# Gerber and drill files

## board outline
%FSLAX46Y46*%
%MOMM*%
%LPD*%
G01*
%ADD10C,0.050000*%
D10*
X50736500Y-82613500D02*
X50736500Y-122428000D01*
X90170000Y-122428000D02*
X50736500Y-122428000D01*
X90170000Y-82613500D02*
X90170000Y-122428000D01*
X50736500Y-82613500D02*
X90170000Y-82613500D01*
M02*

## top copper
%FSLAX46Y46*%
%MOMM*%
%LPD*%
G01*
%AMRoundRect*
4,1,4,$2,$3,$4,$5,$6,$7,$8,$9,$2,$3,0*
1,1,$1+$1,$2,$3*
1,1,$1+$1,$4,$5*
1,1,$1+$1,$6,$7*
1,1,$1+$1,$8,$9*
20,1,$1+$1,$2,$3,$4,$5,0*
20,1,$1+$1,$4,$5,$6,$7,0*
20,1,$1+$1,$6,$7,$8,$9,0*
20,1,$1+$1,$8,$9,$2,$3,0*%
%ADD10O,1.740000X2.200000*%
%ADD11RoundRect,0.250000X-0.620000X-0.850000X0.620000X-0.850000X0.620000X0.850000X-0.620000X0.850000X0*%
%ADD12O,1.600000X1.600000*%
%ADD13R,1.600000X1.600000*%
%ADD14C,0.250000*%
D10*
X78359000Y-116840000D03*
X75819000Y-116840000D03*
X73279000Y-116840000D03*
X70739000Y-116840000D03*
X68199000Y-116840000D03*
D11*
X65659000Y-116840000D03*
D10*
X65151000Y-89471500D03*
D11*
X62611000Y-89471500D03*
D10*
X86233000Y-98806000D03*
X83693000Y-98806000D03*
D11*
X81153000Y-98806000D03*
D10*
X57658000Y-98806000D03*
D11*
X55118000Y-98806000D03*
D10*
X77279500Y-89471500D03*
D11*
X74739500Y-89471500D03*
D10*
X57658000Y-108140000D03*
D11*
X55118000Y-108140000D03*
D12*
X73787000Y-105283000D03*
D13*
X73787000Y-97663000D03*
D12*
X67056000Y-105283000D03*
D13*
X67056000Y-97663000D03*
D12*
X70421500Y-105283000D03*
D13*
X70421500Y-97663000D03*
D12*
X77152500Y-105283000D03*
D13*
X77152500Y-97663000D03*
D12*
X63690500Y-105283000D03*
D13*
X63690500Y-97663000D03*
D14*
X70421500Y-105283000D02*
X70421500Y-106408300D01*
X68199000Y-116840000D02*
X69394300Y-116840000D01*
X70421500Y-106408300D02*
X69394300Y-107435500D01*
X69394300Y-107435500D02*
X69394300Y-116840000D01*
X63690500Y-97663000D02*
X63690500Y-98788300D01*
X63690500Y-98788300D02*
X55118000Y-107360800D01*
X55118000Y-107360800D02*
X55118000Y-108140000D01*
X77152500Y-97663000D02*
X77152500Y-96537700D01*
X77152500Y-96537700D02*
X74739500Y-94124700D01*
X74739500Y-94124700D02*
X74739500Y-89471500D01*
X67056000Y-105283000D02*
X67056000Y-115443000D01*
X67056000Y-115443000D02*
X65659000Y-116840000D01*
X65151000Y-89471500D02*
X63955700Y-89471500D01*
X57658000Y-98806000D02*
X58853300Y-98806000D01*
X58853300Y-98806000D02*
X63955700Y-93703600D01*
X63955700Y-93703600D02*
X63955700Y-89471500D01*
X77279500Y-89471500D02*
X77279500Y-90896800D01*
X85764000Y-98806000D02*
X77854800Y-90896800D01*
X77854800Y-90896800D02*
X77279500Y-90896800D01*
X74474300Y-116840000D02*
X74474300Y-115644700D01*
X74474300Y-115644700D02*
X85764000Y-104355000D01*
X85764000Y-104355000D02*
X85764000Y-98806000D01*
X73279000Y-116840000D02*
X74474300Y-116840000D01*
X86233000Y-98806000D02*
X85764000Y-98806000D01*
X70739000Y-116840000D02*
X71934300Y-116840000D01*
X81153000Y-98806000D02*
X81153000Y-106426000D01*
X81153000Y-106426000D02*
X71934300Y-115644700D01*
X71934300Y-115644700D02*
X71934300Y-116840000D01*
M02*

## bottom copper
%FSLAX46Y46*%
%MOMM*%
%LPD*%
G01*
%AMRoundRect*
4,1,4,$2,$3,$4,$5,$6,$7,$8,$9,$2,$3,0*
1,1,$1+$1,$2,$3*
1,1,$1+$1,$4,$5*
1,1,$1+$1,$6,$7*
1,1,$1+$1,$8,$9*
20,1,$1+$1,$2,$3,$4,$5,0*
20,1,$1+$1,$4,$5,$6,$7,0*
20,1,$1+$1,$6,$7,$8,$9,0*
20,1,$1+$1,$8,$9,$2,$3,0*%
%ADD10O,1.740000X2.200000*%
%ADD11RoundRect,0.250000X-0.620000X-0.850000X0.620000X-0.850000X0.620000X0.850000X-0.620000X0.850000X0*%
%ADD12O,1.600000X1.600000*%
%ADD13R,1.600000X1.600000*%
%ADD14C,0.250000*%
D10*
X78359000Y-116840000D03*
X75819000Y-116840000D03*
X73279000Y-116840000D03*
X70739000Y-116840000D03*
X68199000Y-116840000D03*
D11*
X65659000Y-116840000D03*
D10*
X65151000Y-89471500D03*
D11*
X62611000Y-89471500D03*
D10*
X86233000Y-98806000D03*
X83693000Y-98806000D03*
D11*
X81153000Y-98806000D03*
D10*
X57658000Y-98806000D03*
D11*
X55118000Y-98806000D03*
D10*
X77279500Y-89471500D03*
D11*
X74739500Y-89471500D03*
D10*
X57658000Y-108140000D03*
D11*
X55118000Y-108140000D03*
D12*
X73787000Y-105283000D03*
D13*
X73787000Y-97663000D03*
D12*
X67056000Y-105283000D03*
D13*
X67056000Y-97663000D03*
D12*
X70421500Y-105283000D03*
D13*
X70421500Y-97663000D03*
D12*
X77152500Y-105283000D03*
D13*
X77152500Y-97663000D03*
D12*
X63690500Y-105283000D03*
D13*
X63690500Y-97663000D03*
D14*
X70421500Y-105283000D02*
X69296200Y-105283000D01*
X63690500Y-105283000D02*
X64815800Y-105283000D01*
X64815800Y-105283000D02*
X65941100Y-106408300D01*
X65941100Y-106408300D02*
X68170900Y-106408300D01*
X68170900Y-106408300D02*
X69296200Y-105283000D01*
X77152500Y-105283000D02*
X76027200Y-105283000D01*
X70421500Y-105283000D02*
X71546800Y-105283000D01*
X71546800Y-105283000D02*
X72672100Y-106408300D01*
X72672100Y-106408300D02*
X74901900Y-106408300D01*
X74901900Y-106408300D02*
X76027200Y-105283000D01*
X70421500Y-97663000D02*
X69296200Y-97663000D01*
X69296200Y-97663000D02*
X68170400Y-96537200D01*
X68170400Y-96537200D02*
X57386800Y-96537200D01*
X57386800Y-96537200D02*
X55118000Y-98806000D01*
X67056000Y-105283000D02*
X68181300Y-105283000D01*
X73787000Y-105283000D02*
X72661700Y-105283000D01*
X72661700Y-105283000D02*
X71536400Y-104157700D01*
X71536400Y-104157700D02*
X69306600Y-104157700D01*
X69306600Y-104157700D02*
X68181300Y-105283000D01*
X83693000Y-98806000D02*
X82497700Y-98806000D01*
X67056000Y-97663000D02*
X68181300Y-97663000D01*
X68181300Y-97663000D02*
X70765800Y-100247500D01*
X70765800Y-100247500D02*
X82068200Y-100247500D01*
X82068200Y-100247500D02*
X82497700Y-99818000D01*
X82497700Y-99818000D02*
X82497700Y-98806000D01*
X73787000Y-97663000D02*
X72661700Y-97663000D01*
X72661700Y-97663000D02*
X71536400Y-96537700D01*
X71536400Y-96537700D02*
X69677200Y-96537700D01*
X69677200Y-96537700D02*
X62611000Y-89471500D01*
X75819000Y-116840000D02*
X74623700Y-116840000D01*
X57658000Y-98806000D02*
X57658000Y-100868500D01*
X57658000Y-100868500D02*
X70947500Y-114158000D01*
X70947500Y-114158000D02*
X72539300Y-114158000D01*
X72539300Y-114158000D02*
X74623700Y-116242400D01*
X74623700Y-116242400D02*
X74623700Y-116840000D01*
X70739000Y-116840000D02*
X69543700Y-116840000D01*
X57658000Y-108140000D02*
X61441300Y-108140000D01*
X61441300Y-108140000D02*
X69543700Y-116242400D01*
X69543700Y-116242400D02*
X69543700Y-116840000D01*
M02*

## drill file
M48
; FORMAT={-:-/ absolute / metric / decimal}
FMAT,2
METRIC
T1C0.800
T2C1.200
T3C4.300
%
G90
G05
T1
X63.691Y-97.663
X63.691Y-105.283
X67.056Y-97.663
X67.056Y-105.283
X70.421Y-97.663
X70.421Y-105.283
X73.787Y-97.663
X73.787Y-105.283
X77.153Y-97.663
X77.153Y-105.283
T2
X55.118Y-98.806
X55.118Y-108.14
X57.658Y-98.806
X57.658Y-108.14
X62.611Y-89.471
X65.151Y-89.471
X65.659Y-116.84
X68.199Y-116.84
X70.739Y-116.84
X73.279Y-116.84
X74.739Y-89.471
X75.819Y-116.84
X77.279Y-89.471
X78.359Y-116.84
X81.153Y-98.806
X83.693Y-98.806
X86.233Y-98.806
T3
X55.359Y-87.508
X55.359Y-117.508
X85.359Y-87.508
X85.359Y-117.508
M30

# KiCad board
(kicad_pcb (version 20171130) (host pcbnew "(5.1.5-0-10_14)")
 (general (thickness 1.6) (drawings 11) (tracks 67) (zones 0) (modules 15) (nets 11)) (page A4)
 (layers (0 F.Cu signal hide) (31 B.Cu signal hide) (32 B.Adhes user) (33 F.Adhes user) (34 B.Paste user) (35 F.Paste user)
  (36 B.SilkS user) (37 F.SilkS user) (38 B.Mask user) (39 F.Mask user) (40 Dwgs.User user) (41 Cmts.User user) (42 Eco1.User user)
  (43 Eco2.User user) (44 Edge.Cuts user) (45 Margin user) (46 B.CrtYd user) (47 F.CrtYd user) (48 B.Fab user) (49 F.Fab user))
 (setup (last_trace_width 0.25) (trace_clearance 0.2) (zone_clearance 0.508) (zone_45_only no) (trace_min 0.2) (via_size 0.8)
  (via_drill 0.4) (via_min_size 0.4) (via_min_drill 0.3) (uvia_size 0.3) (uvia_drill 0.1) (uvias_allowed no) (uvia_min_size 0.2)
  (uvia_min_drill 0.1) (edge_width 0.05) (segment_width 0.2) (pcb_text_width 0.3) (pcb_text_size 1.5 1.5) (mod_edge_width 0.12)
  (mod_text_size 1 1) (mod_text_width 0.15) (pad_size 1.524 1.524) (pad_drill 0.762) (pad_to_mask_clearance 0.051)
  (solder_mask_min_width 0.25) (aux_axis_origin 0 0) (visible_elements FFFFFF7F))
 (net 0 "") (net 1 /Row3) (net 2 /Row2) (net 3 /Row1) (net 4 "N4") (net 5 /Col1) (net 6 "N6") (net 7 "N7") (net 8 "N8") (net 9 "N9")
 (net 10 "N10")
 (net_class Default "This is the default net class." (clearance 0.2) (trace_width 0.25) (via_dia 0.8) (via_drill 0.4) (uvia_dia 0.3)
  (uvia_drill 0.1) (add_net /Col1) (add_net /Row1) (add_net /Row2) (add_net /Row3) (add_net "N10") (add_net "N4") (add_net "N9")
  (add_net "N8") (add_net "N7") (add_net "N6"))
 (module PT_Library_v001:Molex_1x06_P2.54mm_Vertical (layer F.Cu) (at 65.659 116.84)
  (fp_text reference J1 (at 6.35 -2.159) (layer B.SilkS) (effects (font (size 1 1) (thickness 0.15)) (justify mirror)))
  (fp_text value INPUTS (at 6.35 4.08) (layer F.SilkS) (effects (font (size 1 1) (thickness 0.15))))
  (pad 6 thru_hole oval (at 12.7 0) (size 1.74 2.2) (drill 1.2) (layers *.Cu *.Mask))
  (pad 5 thru_hole oval (at 10.16 0) (size 1.74 2.2) (drill 1.2) (layers *.Cu *.Mask) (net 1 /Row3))
  (pad 4 thru_hole oval (at 7.62 0) (size 1.74 2.2) (drill 1.2) (layers *.Cu *.Mask) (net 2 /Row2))
  (pad 3 thru_hole oval (at 5.08 0) (size 1.74 2.2) (drill 1.2) (layers *.Cu *.Mask) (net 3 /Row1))
  (pad 2 thru_hole oval (at 2.54 0) (size 1.74 2.2) (drill 1.2) (layers *.Cu *.Mask) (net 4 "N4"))
  (pad 1 thru_hole roundrect (at 0 0) (size 1.74 2.2) (drill 1.2) (layers *.Cu *.Mask) (roundrect_rratio 0.143678) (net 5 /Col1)))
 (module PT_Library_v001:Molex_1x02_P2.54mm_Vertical (layer F.Cu) (at 62.611 89.4715)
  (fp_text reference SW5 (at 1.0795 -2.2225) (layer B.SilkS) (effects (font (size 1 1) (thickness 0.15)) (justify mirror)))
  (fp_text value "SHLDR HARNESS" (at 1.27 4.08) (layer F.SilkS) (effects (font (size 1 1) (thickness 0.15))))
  (pad 2 thru_hole oval (at 2.54 0) (size 1.74 2.2) (drill 1.2) (layers *.Cu *.Mask) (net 1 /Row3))
  (pad 1 thru_hole roundrect (at 0 0) (size 1.74 2.2) (drill 1.2) (layers *.Cu *.Mask) (roundrect_rratio 0.143678) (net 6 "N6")))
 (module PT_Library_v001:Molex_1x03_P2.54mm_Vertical (layer F.Cu) (at 81.153 98.806)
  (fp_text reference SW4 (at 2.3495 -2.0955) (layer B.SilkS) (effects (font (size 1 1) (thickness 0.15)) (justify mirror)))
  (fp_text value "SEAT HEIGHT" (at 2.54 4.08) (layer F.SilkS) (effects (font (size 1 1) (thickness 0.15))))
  (pad 3 thru_hole oval (at 5.08 0) (size 1.74 2.2) (drill 1.2) (layers *.Cu *.Mask) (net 2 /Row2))
  (pad 2 thru_hole oval (at 2.54 0) (size 1.74 2.2) (drill 1.2) (layers *.Cu *.Mask) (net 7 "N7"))
  (pad 1 thru_hole roundrect (at 0 0) (size 1.74 2.2) (drill 1.2) (layers *.Cu *.Mask) (roundrect_rratio 0.143678) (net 3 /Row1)))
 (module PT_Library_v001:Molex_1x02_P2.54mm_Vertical (layer F.Cu) (at 55.118 98.806)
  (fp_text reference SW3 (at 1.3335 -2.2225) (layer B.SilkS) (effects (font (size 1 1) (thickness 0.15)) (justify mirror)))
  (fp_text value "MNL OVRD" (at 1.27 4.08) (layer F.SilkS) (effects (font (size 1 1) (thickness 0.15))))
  (pad 2 thru_hole oval (at 2.54 0) (size 1.74 2.2) (drill 1.2) (layers *.Cu *.Mask) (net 1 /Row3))
  (pad 1 thru_hole roundrect (at 0 0) (size 1.74 2.2) (drill 1.2) (layers *.Cu *.Mask) (roundrect_rratio 0.143678) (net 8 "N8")))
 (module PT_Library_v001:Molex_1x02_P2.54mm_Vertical (layer F.Cu) (at 74.7395 89.4715)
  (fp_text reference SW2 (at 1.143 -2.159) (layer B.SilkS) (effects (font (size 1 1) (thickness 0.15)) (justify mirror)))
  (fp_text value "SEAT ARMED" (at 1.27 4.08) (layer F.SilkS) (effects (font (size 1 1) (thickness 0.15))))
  (pad 2 thru_hole oval (at 2.54 0) (size 1.74 2.2) (drill 1.2) (layers *.Cu *.Mask) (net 2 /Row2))
  (pad 1 thru_hole roundrect (at 0 0) (size 1.74 2.2) (drill 1.2) (layers *.Cu *.Mask) (roundrect_rratio 0.143678) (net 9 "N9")))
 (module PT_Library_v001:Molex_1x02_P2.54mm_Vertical (layer F.Cu) (at 55.118 108.14)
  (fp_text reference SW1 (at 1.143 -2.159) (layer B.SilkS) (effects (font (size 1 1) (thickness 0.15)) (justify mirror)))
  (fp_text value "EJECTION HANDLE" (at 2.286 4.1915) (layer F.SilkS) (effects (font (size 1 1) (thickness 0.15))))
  (pad 2 thru_hole oval (at 2.54 0) (size 1.74 2.2) (drill 1.2) (layers *.Cu *.Mask) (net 3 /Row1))
  (pad 1 thru_hole roundrect (at 0 0) (size 1.74 2.2) (drill 1.2) (layers *.Cu *.Mask) (roundrect_rratio 0.143678) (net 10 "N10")))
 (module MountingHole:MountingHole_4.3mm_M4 (layer F.Cu) (at 55.3595 117.508)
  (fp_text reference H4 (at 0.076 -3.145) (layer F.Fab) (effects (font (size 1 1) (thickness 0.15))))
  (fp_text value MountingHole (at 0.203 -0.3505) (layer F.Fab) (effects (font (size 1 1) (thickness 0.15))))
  (pad 1 np_thru_hole circle (at 0 0) (size 4.3 4.3) (drill 4.3) (layers *.Cu *.Mask)))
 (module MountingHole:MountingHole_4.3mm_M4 (layer F.Cu) (at 85.3595 117.508)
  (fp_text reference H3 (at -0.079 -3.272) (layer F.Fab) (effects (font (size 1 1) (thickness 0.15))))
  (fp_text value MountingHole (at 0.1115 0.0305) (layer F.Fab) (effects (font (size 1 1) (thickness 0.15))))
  (pad 1 np_thru_hole circle (at 0 0) (size 4.3 4.3) (drill 4.3) (layers *.Cu *.Mask)))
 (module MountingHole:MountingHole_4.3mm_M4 (layer F.Cu) (at 55.3595 87.5085)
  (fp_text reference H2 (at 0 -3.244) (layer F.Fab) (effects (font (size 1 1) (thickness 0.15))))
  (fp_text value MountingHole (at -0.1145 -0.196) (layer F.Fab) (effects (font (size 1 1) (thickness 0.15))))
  (pad 1 np_thru_hole circle (at 0 0) (size 4.3 4.3) (drill 4.3) (layers *.Cu *.Mask)))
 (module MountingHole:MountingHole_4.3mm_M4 (layer F.Cu) (at 85.3595 87.5085)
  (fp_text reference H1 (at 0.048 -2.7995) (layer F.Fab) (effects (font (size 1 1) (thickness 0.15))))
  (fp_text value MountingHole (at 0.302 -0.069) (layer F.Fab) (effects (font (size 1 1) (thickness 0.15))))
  (pad 1 np_thru_hole circle (at 0 0) (size 4.3 4.3) (drill 4.3) (layers *.Cu *.Mask)))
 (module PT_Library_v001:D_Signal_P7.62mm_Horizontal (layer F.Cu) (at 73.787 97.663 270)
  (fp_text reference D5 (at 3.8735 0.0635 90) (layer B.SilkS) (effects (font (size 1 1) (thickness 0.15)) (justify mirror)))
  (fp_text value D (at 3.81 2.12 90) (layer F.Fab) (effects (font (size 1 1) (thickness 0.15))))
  (pad 2 thru_hole oval (at 7.62 0 270) (size 1.6 1.6) (drill 0.8) (layers *.Cu *.Mask) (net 5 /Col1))
  (pad 1 thru_hole rect (at 0 0 270) (size 1.6 1.6) (drill 0.8) (layers *.Cu *.Mask) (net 6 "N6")))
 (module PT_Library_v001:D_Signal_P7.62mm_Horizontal (layer F.Cu) (at 67.056 97.663 270)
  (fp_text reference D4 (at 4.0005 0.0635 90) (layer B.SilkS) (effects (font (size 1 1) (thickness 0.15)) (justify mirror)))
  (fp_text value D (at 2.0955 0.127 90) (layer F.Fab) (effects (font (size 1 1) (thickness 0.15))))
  (pad 2 thru_hole oval (at 7.62 0 270) (size 1.6 1.6) (drill 0.8) (layers *.Cu *.Mask) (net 5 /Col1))
  (pad 1 thru_hole rect (at 0 0 270) (size 1.6 1.6) (drill 0.8) (layers *.Cu *.Mask) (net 7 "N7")))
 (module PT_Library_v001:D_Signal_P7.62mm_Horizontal (layer F.Cu) (at 70.4215 97.663 270)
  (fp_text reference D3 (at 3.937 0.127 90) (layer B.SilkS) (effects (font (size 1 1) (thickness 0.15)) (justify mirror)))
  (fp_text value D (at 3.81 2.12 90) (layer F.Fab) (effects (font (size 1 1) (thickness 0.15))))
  (pad 2 thru_hole oval (at 7.62 0 270) (size 1.6 1.6) (drill 0.8) (layers *.Cu *.Mask) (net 4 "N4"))
  (pad 1 thru_hole rect (at 0 0 270) (size 1.6 1.6) (drill 0.8) (layers *.Cu *.Mask) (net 8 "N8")))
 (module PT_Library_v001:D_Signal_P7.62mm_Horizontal (layer F.Cu) (at 77.1525 97.663 270)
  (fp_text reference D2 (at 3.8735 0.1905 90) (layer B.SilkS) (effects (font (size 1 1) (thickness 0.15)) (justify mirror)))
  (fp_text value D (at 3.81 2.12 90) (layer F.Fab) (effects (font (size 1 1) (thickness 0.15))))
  (pad 2 thru_hole oval (at 7.62 0 270) (size 1.6 1.6) (drill 0.8) (layers *.Cu *.Mask) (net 4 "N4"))
  (pad 1 thru_hole rect (at 0 0 270) (size 1.6 1.6) (drill 0.8) (layers *.Cu *.Mask) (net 9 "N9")))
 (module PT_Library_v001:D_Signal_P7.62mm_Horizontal (layer F.Cu) (at 63.6905 97.663 270)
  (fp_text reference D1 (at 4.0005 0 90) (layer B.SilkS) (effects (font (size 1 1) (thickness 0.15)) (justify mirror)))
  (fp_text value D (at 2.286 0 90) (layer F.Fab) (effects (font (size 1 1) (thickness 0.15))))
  (pad 2 thru_hole oval (at 7.62 0 270) (size 1.6 1.6) (drill 0.8) (layers *.Cu *.Mask) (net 4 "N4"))
  (pad 1 thru_hole rect (at 0 0 270) (size 1.6 1.6) (drill 0.8) (layers *.Cu *.Mask) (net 10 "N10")))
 (gr_line (start 50.7365 82.6135) (end 50.7365 122.428) (layer Edge.Cuts) (width 0.05))
 (gr_line (start 90.17 122.428) (end 50.7365 122.428) (layer Edge.Cuts) (width 0.05))
 (gr_line (start 90.17 82.6135) (end 90.17 122.428) (layer Edge.Cuts) (width 0.05))
 (gr_line (start 50.7365 82.6135) (end 90.17 82.6135) (layer Edge.Cuts) (width 0.05))
 (segment (start 70.4215 105.283) (end 69.2962 105.283) (width 0.25) (layer B.Cu) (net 4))
 (segment (start 63.6905 105.283) (end 64.8158 105.283) (width 0.25) (layer B.Cu) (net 4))
 (segment (start 64.8158 105.283) (end 65.9411 106.4083) (width 0.25) (layer B.Cu) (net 4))
 (segment (start 65.9411 106.4083) (end 68.1709 106.4083) (width 0.25) (layer B.Cu) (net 4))
 (segment (start 68.1709 106.4083) (end 69.2962 105.283) (width 0.25) (layer B.Cu) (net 4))
 (segment (start 77.1525 105.283) (end 76.0272 105.283) (width 0.25) (layer B.Cu) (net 4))
 (segment (start 70.4215 105.283) (end 71.5468 105.283) (width 0.25) (layer B.Cu) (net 4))
 (segment (start 71.5468 105.283) (end 72.6721 106.4083) (width 0.25) (layer B.Cu) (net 4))
 (segment (start 72.6721 106.4083) (end 74.9019 106.4083) (width 0.25) (layer B.Cu) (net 4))
 (segment (start 74.9019 106.4083) (end 76.0272 105.283) (width 0.25) (layer B.Cu) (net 4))
 (segment (start 70.4215 105.283) (end 70.4215 106.4083) (width 0.25) (layer F.Cu) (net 4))
 (segment (start 68.199 116.84) (end 69.3943 116.84) (width 0.25) (layer F.Cu) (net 4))
 (segment (start 70.4215 106.4083) (end 69.3943 107.4355) (width 0.25) (layer F.Cu) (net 4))
 (segment (start 69.3943 107.4355) (end 69.3943 116.84) (width 0.25) (layer F.Cu) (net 4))
 (segment (start 63.6905 97.663) (end 63.6905 98.7883) (width 0.25) (layer F.Cu) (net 10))
 (segment (start 63.6905 98.7883) (end 55.118 107.3608) (width 0.25) (layer F.Cu) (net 10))
 (segment (start 55.118 107.3608) (end 55.118 108.14) (width 0.25) (layer F.Cu) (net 10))
 (segment (start 77.1525 97.663) (end 77.1525 96.5377) (width 0.25) (layer F.Cu) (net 9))
 (segment (start 77.1525 96.5377) (end 74.7395 94.1247) (width 0.25) (layer F.Cu) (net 9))
 (segment (start 74.7395 94.1247) (end 74.7395 89.4715) (width 0.25) (layer F.Cu) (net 9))
 (segment (start 70.4215 97.663) (end 69.2962 97.663) (width 0.25) (layer B.Cu) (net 8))
 (segment (start 69.2962 97.663) (end 68.1704 96.5372) (width 0.25) (layer B.Cu) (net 8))
 (segment (start 68.1704 96.5372) (end 57.3868 96.5372) (width 0.25) (layer B.Cu) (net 8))
 (segment (start 57.3868 96.5372) (end 55.118 98.806) (width 0.25) (layer B.Cu) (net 8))
 (segment (start 67.056 105.283) (end 68.1813 105.283) (width 0.25) (layer B.Cu) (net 5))
 (segment (start 73.787 105.283) (end 72.6617 105.283) (width 0.25) (layer B.Cu) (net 5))
 (segment (start 72.6617 105.283) (end 71.5364 104.1577) (width 0.25) (layer B.Cu) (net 5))
 (segment (start 71.5364 104.1577) (end 69.3066 104.1577) (width 0.25) (layer B.Cu) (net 5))
 (segment (start 69.3066 104.1577) (end 68.1813 105.283) (width 0.25) (layer B.Cu) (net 5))
 (segment (start 67.056 105.283) (end 67.056 115.443) (width 0.25) (layer F.Cu) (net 5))
 (segment (start 67.056 115.443) (end 65.659 116.84) (width 0.25) (layer F.Cu) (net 5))
 (segment (start 83.693 98.806) (end 82.4977 98.806) (width 0.25) (layer B.Cu) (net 7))
 (segment (start 67.056 97.663) (end 68.1813 97.663) (width 0.25) (layer B.Cu) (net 7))
 (segment (start 68.1813 97.663) (end 70.7658 100.2475) (width 0.25) (layer B.Cu) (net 7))
 (segment (start 70.7658 100.2475) (end 82.0682 100.2475) (width 0.25) (layer B.Cu) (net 7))
 (segment (start 82.0682 100.2475) (end 82.4977 99.818) (width 0.25) (layer B.Cu) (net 7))
 (segment (start 82.4977 99.818) (end 82.4977 98.806) (width 0.25) (layer B.Cu) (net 7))
 (segment (start 73.787 97.663) (end 72.6617 97.663) (width 0.25) (layer B.Cu) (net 6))
 (segment (start 72.6617 97.663) (end 71.5364 96.5377) (width 0.25) (layer B.Cu) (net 6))
 (segment (start 71.5364 96.5377) (end 69.6772 96.5377) (width 0.25) (layer B.Cu) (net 6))
 (segment (start 69.6772 96.5377) (end 62.611 89.4715) (width 0.25) (layer B.Cu) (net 6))
 (segment (start 75.819 116.84) (end 74.6237 116.84) (width 0.25) (layer B.Cu) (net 1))
 (segment (start 57.658 98.806) (end 57.658 100.8685) (width 0.25) (layer B.Cu) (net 1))
 (segment (start 57.658 100.8685) (end 70.9475 114.158) (width 0.25) (layer B.Cu) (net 1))
 (segment (start 70.9475 114.158) (end 72.5393 114.158) (width 0.25) (layer B.Cu) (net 1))
 (segment (start 72.5393 114.158) (end 74.6237 116.2424) (width 0.25) (layer B.Cu) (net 1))
 (segment (start 74.6237 116.2424) (end 74.6237 116.84) (width 0.25) (layer B.Cu) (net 1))
 (segment (start 65.151 89.4715) (end 63.9557 89.4715) (width 0.25) (layer F.Cu) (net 1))
 (segment (start 57.658 98.806) (end 58.8533 98.806) (width 0.25) (layer F.Cu) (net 1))
 (segment (start 58.8533 98.806) (end 63.9557 93.7036) (width 0.25) (layer F.Cu) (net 1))
 (segment (start 63.9557 93.7036) (end 63.9557 89.4715) (width 0.25) (layer F.Cu) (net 1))
 (segment (start 77.2795 89.4715) (end 77.2795 90.8968) (width 0.25) (layer F.Cu) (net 2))
 (segment (start 85.764 98.806) (end 77.8548 90.8968) (width 0.25) (layer F.Cu) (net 2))
 (segment (start 77.8548 90.8968) (end 77.2795 90.8968) (width 0.25) (layer F.Cu) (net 2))
 (segment (start 74.4743 116.84) (end 74.4743 115.6447) (width 0.25) (layer F.Cu) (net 2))
 (segment (start 74.4743 115.6447) (end 85.764 104.355) (width 0.25) (layer F.Cu) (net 2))
 (segment (start 85.764 104.355) (end 85.764 98.806) (width 0.25) (layer F.Cu) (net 2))
 (segment (start 73.279 116.84) (end 74.4743 116.84) (width 0.25) (layer F.Cu) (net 2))
 (segment (start 86.233 98.806) (end 85.764 98.806) (width 0.25) (layer F.Cu) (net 2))
 (segment (start 70.739 116.84) (end 71.9343 116.84) (width 0.25) (layer F.Cu) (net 3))
 (segment (start 81.153 98.806) (end 81.153 106.426) (width 0.25) (layer F.Cu) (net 3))
 (segment (start 81.153 106.426) (end 71.9343 115.6447) (width 0.25) (layer F.Cu) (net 3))
 (segment (start 71.9343 115.6447) (end 71.9343 116.84) (width 0.25) (layer F.Cu) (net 3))
 (segment (start 70.739 116.84) (end 69.5437 116.84) (width 0.25) (layer B.Cu) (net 3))
 (segment (start 57.658 108.14) (end 61.4413 108.14) (width 0.25) (layer B.Cu) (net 3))
 (segment (start 61.4413 108.14) (end 69.5437 116.2424) (width 0.25) (layer B.Cu) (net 3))
 (segment (start 69.5437 116.2424) (end 69.5437 116.84) (width 0.25) (layer B.Cu) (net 3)))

